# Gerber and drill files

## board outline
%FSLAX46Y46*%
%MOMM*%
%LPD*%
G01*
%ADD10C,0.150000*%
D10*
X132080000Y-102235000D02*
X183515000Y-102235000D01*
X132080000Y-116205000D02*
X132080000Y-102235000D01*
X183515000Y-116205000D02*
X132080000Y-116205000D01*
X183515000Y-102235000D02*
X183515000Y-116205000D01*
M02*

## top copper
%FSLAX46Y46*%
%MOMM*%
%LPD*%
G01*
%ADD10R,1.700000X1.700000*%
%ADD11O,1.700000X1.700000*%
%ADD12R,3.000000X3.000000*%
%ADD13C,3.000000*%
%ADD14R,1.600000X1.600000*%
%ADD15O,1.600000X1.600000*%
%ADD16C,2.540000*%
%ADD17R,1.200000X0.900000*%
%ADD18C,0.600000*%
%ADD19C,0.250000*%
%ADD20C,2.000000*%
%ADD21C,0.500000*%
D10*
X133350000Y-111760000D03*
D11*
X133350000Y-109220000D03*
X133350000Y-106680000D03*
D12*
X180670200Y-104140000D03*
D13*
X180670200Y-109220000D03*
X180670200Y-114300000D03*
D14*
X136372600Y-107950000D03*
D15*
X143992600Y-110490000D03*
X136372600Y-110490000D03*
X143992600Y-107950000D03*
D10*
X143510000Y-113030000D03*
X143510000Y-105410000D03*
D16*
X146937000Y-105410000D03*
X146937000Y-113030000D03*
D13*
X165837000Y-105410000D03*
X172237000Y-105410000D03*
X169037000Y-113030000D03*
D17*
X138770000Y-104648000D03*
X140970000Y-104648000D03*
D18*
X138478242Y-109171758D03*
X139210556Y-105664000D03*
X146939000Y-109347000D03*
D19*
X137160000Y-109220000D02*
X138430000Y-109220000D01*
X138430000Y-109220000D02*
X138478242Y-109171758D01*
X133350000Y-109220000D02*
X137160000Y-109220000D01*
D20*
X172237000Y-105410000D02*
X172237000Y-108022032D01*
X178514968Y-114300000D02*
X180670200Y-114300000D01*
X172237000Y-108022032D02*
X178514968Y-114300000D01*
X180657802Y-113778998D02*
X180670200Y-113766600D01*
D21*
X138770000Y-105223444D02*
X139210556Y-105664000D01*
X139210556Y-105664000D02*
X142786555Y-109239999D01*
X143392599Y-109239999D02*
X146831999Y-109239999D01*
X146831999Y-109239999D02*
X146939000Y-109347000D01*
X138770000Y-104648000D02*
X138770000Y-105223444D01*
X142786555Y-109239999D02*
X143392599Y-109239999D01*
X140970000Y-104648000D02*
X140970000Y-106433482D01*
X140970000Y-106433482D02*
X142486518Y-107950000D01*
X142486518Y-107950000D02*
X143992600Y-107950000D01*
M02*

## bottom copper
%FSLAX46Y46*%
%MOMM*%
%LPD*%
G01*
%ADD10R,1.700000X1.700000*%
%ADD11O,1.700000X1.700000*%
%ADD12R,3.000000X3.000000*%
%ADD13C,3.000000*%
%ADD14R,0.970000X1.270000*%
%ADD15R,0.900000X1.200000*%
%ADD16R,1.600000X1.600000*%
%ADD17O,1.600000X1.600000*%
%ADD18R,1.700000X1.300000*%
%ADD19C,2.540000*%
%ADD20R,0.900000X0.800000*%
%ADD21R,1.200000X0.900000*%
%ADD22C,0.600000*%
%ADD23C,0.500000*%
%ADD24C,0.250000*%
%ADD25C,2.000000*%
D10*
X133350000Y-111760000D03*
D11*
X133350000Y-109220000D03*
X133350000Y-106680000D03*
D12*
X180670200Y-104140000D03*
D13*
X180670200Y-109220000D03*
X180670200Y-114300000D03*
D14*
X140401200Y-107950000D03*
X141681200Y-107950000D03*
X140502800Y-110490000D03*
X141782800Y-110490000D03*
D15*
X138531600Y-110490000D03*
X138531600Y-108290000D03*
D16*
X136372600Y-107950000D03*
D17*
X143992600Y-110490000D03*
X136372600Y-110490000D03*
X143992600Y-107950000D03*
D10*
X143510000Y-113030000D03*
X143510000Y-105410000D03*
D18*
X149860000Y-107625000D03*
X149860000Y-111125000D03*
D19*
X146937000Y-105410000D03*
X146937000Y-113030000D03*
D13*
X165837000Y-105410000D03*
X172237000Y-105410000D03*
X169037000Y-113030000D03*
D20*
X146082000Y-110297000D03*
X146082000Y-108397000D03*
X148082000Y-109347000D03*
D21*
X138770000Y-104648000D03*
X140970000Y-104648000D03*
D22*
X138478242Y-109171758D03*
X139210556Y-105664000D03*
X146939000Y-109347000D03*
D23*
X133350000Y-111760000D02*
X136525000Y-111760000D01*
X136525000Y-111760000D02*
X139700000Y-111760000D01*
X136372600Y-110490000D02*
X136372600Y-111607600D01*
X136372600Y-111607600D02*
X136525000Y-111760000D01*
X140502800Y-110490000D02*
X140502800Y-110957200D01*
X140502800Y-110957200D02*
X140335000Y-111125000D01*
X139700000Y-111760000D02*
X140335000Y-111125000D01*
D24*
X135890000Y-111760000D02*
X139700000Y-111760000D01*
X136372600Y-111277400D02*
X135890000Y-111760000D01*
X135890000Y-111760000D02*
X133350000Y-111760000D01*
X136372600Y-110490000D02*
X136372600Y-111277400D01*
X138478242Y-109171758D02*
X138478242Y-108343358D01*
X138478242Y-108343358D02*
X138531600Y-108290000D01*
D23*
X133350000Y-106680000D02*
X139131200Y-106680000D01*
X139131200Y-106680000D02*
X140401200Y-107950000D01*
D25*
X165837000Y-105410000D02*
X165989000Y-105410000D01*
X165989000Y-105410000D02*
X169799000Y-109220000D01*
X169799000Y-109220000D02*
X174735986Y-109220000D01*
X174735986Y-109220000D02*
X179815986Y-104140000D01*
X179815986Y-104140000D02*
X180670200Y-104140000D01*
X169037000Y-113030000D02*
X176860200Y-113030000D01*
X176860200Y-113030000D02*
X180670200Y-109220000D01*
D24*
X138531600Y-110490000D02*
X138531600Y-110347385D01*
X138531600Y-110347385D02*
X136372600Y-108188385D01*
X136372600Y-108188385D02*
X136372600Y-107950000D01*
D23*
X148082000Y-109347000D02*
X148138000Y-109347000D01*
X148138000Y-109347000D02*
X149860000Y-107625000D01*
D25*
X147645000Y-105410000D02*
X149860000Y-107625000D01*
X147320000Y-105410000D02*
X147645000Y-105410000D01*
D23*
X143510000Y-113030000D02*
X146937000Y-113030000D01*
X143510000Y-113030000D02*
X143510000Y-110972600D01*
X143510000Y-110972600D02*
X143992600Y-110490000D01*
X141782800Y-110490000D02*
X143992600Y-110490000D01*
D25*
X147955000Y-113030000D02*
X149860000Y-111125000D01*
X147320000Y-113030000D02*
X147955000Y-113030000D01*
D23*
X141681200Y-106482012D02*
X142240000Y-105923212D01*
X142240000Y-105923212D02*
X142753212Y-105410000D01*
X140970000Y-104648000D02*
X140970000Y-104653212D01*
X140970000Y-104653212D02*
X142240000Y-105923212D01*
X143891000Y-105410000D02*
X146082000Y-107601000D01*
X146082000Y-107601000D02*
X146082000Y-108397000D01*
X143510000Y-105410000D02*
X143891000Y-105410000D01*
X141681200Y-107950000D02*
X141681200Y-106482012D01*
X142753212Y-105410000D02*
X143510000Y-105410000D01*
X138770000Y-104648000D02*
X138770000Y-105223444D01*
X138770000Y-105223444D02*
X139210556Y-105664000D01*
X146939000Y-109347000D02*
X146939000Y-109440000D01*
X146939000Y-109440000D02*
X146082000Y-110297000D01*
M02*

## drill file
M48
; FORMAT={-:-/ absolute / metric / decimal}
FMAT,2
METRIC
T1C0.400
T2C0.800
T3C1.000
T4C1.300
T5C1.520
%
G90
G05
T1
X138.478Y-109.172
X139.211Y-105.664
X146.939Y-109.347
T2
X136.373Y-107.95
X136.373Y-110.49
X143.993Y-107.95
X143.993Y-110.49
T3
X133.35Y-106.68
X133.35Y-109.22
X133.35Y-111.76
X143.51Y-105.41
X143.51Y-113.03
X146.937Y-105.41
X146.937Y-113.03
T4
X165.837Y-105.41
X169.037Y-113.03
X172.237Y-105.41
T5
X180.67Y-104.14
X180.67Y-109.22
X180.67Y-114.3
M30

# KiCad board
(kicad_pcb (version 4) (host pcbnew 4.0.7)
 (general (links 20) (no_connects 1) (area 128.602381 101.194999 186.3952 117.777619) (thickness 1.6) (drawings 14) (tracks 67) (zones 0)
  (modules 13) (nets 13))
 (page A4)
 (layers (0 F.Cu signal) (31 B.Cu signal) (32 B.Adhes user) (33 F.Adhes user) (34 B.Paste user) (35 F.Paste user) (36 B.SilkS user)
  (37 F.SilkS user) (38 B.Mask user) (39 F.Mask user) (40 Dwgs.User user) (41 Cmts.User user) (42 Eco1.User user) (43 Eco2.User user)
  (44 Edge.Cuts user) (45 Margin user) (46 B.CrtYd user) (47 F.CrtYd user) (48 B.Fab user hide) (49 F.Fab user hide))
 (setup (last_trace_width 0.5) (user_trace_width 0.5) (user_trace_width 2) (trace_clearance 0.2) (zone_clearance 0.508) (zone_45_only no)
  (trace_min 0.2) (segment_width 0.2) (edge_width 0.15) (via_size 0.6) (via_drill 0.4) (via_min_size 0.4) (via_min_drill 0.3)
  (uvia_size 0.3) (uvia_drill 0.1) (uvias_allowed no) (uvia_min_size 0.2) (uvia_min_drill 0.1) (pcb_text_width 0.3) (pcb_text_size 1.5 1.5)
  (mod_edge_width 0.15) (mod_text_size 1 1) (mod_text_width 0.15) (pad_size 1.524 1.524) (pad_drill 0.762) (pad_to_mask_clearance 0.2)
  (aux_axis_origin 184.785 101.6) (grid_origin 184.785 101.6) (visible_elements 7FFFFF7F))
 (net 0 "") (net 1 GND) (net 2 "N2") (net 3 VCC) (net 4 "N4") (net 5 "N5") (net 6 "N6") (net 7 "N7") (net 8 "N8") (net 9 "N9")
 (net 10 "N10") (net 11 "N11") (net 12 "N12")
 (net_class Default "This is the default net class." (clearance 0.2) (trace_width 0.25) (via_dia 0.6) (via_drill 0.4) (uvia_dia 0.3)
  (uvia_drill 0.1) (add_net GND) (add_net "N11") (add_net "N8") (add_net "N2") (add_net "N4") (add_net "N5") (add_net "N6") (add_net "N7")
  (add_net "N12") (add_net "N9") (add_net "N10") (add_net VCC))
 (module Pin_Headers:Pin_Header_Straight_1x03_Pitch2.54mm (layer F.Cu) (at 133.35 111.76 180)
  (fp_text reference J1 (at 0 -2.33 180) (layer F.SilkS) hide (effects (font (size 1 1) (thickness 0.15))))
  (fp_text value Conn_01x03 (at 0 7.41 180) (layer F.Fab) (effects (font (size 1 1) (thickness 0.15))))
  (pad 1 thru_hole rect (at 0 0 180) (size 1.7 1.7) (drill 1) (layers *.Cu *.Mask) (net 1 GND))
  (pad 2 thru_hole oval (at 0 2.54 180) (size 1.7 1.7) (drill 1) (layers *.Cu *.Mask) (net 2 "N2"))
  (pad 3 thru_hole oval (at 0 5.08 180) (size 1.7 1.7) (drill 1) (layers *.Cu *.Mask) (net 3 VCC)))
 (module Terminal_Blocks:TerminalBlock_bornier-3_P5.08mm (layer F.Cu) (at 180.6702 104.14 270)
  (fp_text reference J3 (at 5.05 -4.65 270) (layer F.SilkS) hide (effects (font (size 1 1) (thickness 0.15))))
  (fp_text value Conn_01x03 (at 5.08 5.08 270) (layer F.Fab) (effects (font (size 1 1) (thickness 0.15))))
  (pad 1 thru_hole rect (at 0 0 270) (size 3 3) (drill 1.52) (layers *.Cu *.Mask) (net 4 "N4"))
  (pad 2 thru_hole circle (at 5.08 0 270) (size 3 3) (drill 1.52) (layers *.Cu *.Mask) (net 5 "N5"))
  (pad 3 thru_hole circle (at 10.16 0 270) (size 3 3) (drill 1.52) (layers *.Cu *.Mask) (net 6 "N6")))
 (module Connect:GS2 (layer B.Cu) (at 141.0412 107.95 270)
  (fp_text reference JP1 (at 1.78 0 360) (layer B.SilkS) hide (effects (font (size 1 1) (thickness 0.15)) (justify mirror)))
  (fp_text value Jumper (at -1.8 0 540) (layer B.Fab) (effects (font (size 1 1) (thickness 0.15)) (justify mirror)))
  (pad 1 smd rect (at 0 0.64 270) (size 1.27 0.97) (layers B.Cu B.Paste B.Mask) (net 3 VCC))
  (pad 2 smd rect (at 0 -0.64 270) (size 1.27 0.97) (layers B.Cu B.Paste B.Mask) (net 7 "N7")))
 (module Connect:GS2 (layer B.Cu) (at 141.1428 110.49 270)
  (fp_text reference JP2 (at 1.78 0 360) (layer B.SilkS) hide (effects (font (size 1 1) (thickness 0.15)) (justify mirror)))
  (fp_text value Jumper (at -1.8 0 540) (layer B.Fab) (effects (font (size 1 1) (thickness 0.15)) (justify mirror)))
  (pad 1 smd rect (at 0 0.64 270) (size 1.27 0.97) (layers B.Cu B.Paste B.Mask) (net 1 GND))
  (pad 2 smd rect (at 0 -0.64 270) (size 1.27 0.97) (layers B.Cu B.Paste B.Mask) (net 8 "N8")))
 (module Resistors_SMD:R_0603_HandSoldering (layer B.Cu) (at 138.5316 109.39 90)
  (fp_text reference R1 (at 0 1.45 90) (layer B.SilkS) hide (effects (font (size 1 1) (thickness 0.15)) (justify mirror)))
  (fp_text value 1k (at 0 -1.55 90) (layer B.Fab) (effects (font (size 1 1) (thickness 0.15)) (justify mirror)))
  (pad 1 smd rect (at -1.1 0 90) (size 1.2 0.9) (layers B.Cu B.Paste B.Mask) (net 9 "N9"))
  (pad 2 smd rect (at 1.1 0 90) (size 1.2 0.9) (layers B.Cu B.Paste B.Mask) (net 2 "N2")))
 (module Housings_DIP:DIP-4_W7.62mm (layer F.Cu) (at 136.3726 107.95)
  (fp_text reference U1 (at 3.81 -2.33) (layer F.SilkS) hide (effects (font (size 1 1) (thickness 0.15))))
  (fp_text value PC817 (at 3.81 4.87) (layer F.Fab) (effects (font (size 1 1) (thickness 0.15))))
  (pad 1 thru_hole rect (at 0 0) (size 1.6 1.6) (drill 0.8) (layers *.Cu *.Mask) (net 9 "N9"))
  (pad 3 thru_hole oval (at 7.62 2.54) (size 1.6 1.6) (drill 0.8) (layers *.Cu *.Mask) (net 8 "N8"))
  (pad 2 thru_hole oval (at 0 2.54) (size 1.6 1.6) (drill 0.8) (layers *.Cu *.Mask) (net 1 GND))
  (pad 4 thru_hole oval (at 7.62 0) (size 1.6 1.6) (drill 0.8) (layers *.Cu *.Mask) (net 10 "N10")))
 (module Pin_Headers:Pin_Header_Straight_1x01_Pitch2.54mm (layer F.Cu) (at 143.51 113.03 90)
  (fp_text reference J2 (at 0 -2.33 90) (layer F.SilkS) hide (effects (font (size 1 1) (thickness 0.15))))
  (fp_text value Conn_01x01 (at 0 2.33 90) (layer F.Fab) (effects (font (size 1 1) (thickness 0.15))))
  (pad 1 thru_hole rect (at 0 0 90) (size 1.7 1.7) (drill 1) (layers *.Cu *.Mask) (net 8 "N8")))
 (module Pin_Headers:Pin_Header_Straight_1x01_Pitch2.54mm (layer F.Cu) (at 143.51 105.41)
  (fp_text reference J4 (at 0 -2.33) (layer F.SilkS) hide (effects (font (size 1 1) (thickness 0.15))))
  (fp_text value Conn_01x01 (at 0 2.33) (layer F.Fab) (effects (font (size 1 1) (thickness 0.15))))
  (pad 1 thru_hole rect (at 0 0) (size 1.7 1.7) (drill 1) (layers *.Cu *.Mask) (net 7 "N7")))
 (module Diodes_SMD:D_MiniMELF (layer B.Cu) (at 149.86 109.375 270)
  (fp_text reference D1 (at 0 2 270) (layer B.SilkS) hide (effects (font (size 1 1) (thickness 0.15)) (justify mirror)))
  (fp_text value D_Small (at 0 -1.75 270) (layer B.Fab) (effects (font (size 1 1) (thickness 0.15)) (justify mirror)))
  (pad 1 smd rect (at -1.75 0 270) (size 1.3 1.7) (layers B.Cu B.Paste B.Mask) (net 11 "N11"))
  (pad 2 smd rect (at 1.75 0 270) (size 1.3 1.7) (layers B.Cu B.Paste B.Mask) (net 8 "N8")))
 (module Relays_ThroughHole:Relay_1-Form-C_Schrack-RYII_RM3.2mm (layer F.Cu) (at 146.937 113.03)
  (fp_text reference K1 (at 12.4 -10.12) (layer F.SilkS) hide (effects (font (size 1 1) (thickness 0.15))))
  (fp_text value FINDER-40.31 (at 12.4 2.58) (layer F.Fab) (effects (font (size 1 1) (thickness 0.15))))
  (pad A2 thru_hole circle (at 0 -7.62) (size 2.54 2.54) (drill 1) (layers *.Cu *.Mask) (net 11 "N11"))
  (pad A1 thru_hole circle (at 0 0) (size 2.54 2.54) (drill 1) (layers *.Cu *.Mask) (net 8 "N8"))
  (pad 12 thru_hole circle (at 18.9 -7.62) (size 3 3) (drill 1.3) (layers *.Cu *.Mask) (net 4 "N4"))
  (pad 14 thru_hole circle (at 25.3 -7.62) (size 3 3) (drill 1.3) (layers *.Cu *.Mask) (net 6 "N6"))
  (pad 11 thru_hole circle (at 22.1 0) (size 3 3) (drill 1.3) (layers *.Cu *.Mask) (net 5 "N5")))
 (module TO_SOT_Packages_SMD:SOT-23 (layer B.Cu) (at 147.082 109.347)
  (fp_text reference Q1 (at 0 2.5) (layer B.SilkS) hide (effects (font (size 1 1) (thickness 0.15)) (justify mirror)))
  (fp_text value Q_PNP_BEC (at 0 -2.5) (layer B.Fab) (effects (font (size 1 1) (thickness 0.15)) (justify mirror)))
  (pad 1 smd rect (at -1 0.95) (size 0.9 0.8) (layers B.Cu B.Paste B.Mask) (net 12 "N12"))
  (pad 2 smd rect (at -1 -0.95) (size 0.9 0.8) (layers B.Cu B.Paste B.Mask) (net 7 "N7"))
  (pad 3 smd rect (at 1 0) (size 0.9 0.8) (layers B.Cu B.Paste B.Mask) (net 11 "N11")))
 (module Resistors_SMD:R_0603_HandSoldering (layer F.Cu) (at 139.87 104.648)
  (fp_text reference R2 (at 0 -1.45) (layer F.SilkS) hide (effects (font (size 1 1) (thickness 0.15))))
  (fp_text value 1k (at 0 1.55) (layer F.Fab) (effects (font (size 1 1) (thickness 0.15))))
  (pad 1 smd rect (at -1.1 0) (size 1.2 0.9) (layers F.Cu F.Paste F.Mask) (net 12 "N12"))
  (pad 2 smd rect (at 1.1 0) (size 1.2 0.9) (layers F.Cu F.Paste F.Mask) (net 10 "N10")))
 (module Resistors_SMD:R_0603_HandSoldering (layer B.Cu) (at 139.87 104.648)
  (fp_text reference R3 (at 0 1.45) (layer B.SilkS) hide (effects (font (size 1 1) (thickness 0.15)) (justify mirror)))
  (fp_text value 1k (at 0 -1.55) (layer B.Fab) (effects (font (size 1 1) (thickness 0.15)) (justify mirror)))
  (pad 1 smd rect (at -1.1 0) (size 1.2 0.9) (layers B.Cu B.Paste B.Mask) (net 12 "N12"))
  (pad 2 smd rect (at 1.1 0) (size 1.2 0.9) (layers B.Cu B.Paste B.Mask) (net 7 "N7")))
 (gr_line (start 132.08 102.235) (end 183.515 102.235) (layer Edge.Cuts) (width 0.15))
 (gr_line (start 132.08 116.205) (end 132.08 102.235) (layer Edge.Cuts) (width 0.15))
 (gr_line (start 183.515 116.205) (end 132.08 116.205) (layer Edge.Cuts) (width 0.15))
 (gr_line (start 183.515 102.235) (end 183.515 116.205) (layer Edge.Cuts) (width 0.15))
 (segment (start 133.35 111.76) (end 136.525 111.76) (width 0.5) (layer B.Cu) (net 1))
 (segment (start 136.525 111.76) (end 139.7 111.76) (width 0.5) (layer B.Cu) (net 1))
 (segment (start 136.3726 110.49) (end 136.3726 111.6076) (width 0.5) (layer B.Cu) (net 1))
 (segment (start 136.3726 111.6076) (end 136.525 111.76) (width 0.5) (layer B.Cu) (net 1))
 (segment (start 140.5028 110.49) (end 140.5028 110.9572) (width 0.5) (layer B.Cu) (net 1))
 (segment (start 140.5028 110.9572) (end 140.335 111.125) (width 0.5) (layer B.Cu) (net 1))
 (segment (start 139.7 111.76) (end 140.335 111.125) (width 0.5) (layer B.Cu) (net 1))
 (segment (start 135.89 111.76) (end 139.7 111.76) (width 0.25) (layer B.Cu) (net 1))
 (segment (start 136.3726 111.2774) (end 135.89 111.76) (width 0.25) (layer B.Cu) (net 1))
 (segment (start 135.89 111.76) (end 133.35 111.76) (width 0.25) (layer B.Cu) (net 1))
 (segment (start 136.3726 110.49) (end 136.3726 111.2774) (width 0.25) (layer B.Cu) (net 1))
 (segment (start 138.478242 109.171758) (end 138.478242 108.343358) (width 0.25) (layer B.Cu) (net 2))
 (segment (start 138.478242 108.343358) (end 138.5316 108.29) (width 0.25) (layer B.Cu) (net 2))
 (segment (start 137.16 109.22) (end 138.43 109.22) (width 0.25) (layer F.Cu) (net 2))
 (segment (start 138.43 109.22) (end 138.478242 109.171758) (width 0.25) (layer F.Cu) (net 2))
 (via (at 138.478242 109.171758) (size 0.6) (drill 0.4) (layers F.Cu B.Cu) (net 2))
 (segment (start 133.35 109.22) (end 137.16 109.22) (width 0.25) (layer F.Cu) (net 2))
 (segment (start 133.35 106.68) (end 139.1312 106.68) (width 0.5) (layer B.Cu) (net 3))
 (segment (start 139.1312 106.68) (end 140.4012 107.95) (width 0.5) (layer B.Cu) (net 3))
 (segment (start 165.837 105.41) (end 165.989 105.41) (width 2) (layer B.Cu) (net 4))
 (segment (start 165.989 105.41) (end 169.799 109.22) (width 2) (layer B.Cu) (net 4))
 (segment (start 169.799 109.22) (end 174.735986 109.22) (width 2) (layer B.Cu) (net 4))
 (segment (start 174.735986 109.22) (end 179.815986 104.14) (width 2) (layer B.Cu) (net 4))
 (segment (start 179.815986 104.14) (end 180.6702 104.14) (width 2) (layer B.Cu) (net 4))
 (segment (start 169.037 113.03) (end 176.8602 113.03) (width 2) (layer B.Cu) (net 5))
 (segment (start 176.8602 113.03) (end 180.6702 109.22) (width 2) (layer B.Cu) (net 5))
 (segment (start 172.237 105.41) (end 172.237 108.022032) (width 2) (layer F.Cu) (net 6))
 (segment (start 178.514968 114.3) (end 180.6702 114.3) (width 2) (layer F.Cu) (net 6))
 (segment (start 172.237 108.022032) (end 178.514968 114.3) (width 2) (layer F.Cu) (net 6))
 (segment (start 180.657802 113.778998) (end 180.6702 113.7666) (width 2) (layer F.Cu) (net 6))
 (segment (start 138.5316 110.49) (end 138.5316 110.347385) (width 0.25) (layer B.Cu) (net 9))
 (segment (start 138.5316 110.347385) (end 136.3726 108.188385) (width 0.25) (layer B.Cu) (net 9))
 (segment (start 136.3726 108.188385) (end 136.3726 107.95) (width 0.25) (layer B.Cu) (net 9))
 (segment (start 148.082 109.347) (end 148.138 109.347) (width 0.5) (layer B.Cu) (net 11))
 (segment (start 148.138 109.347) (end 149.86 107.625) (width 0.5) (layer B.Cu) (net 11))
 (segment (start 147.645 105.41) (end 149.86 107.625) (width 2) (layer B.Cu) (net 11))
 (segment (start 147.32 105.41) (end 147.645 105.41) (width 2) (layer B.Cu) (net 11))
 (segment (start 143.51 113.03) (end 146.937 113.03) (width 0.5) (layer B.Cu) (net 8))
 (segment (start 143.51 113.03) (end 143.51 110.9726) (width 0.5) (layer B.Cu) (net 8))
 (segment (start 143.51 110.9726) (end 143.9926 110.49) (width 0.5) (layer B.Cu) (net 8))
 (segment (start 141.7828 110.49) (end 143.9926 110.49) (width 0.5) (layer B.Cu) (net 8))
 (segment (start 147.955 113.03) (end 149.86 111.125) (width 2) (layer B.Cu) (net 8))
 (segment (start 147.32 113.03) (end 147.955 113.03) (width 2) (layer B.Cu) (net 8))
 (segment (start 141.6812 106.482012) (end 142.24 105.923212) (width 0.5) (layer B.Cu) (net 7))
 (segment (start 142.24 105.923212) (end 142.753212 105.41) (width 0.5) (layer B.Cu) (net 7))
 (segment (start 140.97 104.648) (end 140.97 104.653212) (width 0.5) (layer B.Cu) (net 7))
 (segment (start 140.97 104.653212) (end 142.24 105.923212) (width 0.5) (layer B.Cu) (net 7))
 (segment (start 143.891 105.41) (end 146.082 107.601) (width 0.5) (layer B.Cu) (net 7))
 (segment (start 146.082 107.601) (end 146.082 108.397) (width 0.5) (layer B.Cu) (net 7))
 (segment (start 143.51 105.41) (end 143.891 105.41) (width 0.5) (layer B.Cu) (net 7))
 (segment (start 141.6812 107.95) (end 141.6812 106.482012) (width 0.5) (layer B.Cu) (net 7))
 (segment (start 142.753212 105.41) (end 143.51 105.41) (width 0.5) (layer B.Cu) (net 7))
 (segment (start 138.77 105.223444) (end 139.210556 105.664) (width 0.5) (layer F.Cu) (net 12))
 (segment (start 139.210556 105.664) (end 142.786555 109.239999) (width 0.5) (layer F.Cu) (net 12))
 (via (at 139.210556 105.664) (size 0.6) (drill 0.4) (layers F.Cu B.Cu) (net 12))
 (segment (start 138.77 104.648) (end 138.77 105.223444) (width 0.5) (layer B.Cu) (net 12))
 (segment (start 138.77 105.223444) (end 139.210556 105.664) (width 0.5) (layer B.Cu) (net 12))
 (segment (start 146.939 109.347) (end 146.939 109.44) (width 0.5) (layer B.Cu) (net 12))
 (segment (start 146.939 109.44) (end 146.082 110.297) (width 0.5) (layer B.Cu) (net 12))
 (segment (start 143.392599 109.239999) (end 146.831999 109.239999) (width 0.5) (layer F.Cu) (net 12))
 (segment (start 146.831999 109.239999) (end 146.939 109.347) (width 0.5) (layer F.Cu) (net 12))
 (via (at 146.939 109.347) (size 0.6) (drill 0.4) (layers F.Cu B.Cu) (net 12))
 (segment (start 138.77 104.648) (end 138.77 105.223444) (width 0.5) (layer F.Cu) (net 12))
 (segment (start 142.786555 109.239999) (end 143.392599 109.239999) (width 0.5) (layer F.Cu) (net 12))
 (segment (start 140.97 104.648) (end 140.97 106.433482) (width 0.5) (layer F.Cu) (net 10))
 (segment (start 140.97 106.433482) (end 142.486518 107.95) (width 0.5) (layer F.Cu) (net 10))
 (segment (start 142.486518 107.95) (end 143.9926 107.95) (width 0.5) (layer F.Cu) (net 10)))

